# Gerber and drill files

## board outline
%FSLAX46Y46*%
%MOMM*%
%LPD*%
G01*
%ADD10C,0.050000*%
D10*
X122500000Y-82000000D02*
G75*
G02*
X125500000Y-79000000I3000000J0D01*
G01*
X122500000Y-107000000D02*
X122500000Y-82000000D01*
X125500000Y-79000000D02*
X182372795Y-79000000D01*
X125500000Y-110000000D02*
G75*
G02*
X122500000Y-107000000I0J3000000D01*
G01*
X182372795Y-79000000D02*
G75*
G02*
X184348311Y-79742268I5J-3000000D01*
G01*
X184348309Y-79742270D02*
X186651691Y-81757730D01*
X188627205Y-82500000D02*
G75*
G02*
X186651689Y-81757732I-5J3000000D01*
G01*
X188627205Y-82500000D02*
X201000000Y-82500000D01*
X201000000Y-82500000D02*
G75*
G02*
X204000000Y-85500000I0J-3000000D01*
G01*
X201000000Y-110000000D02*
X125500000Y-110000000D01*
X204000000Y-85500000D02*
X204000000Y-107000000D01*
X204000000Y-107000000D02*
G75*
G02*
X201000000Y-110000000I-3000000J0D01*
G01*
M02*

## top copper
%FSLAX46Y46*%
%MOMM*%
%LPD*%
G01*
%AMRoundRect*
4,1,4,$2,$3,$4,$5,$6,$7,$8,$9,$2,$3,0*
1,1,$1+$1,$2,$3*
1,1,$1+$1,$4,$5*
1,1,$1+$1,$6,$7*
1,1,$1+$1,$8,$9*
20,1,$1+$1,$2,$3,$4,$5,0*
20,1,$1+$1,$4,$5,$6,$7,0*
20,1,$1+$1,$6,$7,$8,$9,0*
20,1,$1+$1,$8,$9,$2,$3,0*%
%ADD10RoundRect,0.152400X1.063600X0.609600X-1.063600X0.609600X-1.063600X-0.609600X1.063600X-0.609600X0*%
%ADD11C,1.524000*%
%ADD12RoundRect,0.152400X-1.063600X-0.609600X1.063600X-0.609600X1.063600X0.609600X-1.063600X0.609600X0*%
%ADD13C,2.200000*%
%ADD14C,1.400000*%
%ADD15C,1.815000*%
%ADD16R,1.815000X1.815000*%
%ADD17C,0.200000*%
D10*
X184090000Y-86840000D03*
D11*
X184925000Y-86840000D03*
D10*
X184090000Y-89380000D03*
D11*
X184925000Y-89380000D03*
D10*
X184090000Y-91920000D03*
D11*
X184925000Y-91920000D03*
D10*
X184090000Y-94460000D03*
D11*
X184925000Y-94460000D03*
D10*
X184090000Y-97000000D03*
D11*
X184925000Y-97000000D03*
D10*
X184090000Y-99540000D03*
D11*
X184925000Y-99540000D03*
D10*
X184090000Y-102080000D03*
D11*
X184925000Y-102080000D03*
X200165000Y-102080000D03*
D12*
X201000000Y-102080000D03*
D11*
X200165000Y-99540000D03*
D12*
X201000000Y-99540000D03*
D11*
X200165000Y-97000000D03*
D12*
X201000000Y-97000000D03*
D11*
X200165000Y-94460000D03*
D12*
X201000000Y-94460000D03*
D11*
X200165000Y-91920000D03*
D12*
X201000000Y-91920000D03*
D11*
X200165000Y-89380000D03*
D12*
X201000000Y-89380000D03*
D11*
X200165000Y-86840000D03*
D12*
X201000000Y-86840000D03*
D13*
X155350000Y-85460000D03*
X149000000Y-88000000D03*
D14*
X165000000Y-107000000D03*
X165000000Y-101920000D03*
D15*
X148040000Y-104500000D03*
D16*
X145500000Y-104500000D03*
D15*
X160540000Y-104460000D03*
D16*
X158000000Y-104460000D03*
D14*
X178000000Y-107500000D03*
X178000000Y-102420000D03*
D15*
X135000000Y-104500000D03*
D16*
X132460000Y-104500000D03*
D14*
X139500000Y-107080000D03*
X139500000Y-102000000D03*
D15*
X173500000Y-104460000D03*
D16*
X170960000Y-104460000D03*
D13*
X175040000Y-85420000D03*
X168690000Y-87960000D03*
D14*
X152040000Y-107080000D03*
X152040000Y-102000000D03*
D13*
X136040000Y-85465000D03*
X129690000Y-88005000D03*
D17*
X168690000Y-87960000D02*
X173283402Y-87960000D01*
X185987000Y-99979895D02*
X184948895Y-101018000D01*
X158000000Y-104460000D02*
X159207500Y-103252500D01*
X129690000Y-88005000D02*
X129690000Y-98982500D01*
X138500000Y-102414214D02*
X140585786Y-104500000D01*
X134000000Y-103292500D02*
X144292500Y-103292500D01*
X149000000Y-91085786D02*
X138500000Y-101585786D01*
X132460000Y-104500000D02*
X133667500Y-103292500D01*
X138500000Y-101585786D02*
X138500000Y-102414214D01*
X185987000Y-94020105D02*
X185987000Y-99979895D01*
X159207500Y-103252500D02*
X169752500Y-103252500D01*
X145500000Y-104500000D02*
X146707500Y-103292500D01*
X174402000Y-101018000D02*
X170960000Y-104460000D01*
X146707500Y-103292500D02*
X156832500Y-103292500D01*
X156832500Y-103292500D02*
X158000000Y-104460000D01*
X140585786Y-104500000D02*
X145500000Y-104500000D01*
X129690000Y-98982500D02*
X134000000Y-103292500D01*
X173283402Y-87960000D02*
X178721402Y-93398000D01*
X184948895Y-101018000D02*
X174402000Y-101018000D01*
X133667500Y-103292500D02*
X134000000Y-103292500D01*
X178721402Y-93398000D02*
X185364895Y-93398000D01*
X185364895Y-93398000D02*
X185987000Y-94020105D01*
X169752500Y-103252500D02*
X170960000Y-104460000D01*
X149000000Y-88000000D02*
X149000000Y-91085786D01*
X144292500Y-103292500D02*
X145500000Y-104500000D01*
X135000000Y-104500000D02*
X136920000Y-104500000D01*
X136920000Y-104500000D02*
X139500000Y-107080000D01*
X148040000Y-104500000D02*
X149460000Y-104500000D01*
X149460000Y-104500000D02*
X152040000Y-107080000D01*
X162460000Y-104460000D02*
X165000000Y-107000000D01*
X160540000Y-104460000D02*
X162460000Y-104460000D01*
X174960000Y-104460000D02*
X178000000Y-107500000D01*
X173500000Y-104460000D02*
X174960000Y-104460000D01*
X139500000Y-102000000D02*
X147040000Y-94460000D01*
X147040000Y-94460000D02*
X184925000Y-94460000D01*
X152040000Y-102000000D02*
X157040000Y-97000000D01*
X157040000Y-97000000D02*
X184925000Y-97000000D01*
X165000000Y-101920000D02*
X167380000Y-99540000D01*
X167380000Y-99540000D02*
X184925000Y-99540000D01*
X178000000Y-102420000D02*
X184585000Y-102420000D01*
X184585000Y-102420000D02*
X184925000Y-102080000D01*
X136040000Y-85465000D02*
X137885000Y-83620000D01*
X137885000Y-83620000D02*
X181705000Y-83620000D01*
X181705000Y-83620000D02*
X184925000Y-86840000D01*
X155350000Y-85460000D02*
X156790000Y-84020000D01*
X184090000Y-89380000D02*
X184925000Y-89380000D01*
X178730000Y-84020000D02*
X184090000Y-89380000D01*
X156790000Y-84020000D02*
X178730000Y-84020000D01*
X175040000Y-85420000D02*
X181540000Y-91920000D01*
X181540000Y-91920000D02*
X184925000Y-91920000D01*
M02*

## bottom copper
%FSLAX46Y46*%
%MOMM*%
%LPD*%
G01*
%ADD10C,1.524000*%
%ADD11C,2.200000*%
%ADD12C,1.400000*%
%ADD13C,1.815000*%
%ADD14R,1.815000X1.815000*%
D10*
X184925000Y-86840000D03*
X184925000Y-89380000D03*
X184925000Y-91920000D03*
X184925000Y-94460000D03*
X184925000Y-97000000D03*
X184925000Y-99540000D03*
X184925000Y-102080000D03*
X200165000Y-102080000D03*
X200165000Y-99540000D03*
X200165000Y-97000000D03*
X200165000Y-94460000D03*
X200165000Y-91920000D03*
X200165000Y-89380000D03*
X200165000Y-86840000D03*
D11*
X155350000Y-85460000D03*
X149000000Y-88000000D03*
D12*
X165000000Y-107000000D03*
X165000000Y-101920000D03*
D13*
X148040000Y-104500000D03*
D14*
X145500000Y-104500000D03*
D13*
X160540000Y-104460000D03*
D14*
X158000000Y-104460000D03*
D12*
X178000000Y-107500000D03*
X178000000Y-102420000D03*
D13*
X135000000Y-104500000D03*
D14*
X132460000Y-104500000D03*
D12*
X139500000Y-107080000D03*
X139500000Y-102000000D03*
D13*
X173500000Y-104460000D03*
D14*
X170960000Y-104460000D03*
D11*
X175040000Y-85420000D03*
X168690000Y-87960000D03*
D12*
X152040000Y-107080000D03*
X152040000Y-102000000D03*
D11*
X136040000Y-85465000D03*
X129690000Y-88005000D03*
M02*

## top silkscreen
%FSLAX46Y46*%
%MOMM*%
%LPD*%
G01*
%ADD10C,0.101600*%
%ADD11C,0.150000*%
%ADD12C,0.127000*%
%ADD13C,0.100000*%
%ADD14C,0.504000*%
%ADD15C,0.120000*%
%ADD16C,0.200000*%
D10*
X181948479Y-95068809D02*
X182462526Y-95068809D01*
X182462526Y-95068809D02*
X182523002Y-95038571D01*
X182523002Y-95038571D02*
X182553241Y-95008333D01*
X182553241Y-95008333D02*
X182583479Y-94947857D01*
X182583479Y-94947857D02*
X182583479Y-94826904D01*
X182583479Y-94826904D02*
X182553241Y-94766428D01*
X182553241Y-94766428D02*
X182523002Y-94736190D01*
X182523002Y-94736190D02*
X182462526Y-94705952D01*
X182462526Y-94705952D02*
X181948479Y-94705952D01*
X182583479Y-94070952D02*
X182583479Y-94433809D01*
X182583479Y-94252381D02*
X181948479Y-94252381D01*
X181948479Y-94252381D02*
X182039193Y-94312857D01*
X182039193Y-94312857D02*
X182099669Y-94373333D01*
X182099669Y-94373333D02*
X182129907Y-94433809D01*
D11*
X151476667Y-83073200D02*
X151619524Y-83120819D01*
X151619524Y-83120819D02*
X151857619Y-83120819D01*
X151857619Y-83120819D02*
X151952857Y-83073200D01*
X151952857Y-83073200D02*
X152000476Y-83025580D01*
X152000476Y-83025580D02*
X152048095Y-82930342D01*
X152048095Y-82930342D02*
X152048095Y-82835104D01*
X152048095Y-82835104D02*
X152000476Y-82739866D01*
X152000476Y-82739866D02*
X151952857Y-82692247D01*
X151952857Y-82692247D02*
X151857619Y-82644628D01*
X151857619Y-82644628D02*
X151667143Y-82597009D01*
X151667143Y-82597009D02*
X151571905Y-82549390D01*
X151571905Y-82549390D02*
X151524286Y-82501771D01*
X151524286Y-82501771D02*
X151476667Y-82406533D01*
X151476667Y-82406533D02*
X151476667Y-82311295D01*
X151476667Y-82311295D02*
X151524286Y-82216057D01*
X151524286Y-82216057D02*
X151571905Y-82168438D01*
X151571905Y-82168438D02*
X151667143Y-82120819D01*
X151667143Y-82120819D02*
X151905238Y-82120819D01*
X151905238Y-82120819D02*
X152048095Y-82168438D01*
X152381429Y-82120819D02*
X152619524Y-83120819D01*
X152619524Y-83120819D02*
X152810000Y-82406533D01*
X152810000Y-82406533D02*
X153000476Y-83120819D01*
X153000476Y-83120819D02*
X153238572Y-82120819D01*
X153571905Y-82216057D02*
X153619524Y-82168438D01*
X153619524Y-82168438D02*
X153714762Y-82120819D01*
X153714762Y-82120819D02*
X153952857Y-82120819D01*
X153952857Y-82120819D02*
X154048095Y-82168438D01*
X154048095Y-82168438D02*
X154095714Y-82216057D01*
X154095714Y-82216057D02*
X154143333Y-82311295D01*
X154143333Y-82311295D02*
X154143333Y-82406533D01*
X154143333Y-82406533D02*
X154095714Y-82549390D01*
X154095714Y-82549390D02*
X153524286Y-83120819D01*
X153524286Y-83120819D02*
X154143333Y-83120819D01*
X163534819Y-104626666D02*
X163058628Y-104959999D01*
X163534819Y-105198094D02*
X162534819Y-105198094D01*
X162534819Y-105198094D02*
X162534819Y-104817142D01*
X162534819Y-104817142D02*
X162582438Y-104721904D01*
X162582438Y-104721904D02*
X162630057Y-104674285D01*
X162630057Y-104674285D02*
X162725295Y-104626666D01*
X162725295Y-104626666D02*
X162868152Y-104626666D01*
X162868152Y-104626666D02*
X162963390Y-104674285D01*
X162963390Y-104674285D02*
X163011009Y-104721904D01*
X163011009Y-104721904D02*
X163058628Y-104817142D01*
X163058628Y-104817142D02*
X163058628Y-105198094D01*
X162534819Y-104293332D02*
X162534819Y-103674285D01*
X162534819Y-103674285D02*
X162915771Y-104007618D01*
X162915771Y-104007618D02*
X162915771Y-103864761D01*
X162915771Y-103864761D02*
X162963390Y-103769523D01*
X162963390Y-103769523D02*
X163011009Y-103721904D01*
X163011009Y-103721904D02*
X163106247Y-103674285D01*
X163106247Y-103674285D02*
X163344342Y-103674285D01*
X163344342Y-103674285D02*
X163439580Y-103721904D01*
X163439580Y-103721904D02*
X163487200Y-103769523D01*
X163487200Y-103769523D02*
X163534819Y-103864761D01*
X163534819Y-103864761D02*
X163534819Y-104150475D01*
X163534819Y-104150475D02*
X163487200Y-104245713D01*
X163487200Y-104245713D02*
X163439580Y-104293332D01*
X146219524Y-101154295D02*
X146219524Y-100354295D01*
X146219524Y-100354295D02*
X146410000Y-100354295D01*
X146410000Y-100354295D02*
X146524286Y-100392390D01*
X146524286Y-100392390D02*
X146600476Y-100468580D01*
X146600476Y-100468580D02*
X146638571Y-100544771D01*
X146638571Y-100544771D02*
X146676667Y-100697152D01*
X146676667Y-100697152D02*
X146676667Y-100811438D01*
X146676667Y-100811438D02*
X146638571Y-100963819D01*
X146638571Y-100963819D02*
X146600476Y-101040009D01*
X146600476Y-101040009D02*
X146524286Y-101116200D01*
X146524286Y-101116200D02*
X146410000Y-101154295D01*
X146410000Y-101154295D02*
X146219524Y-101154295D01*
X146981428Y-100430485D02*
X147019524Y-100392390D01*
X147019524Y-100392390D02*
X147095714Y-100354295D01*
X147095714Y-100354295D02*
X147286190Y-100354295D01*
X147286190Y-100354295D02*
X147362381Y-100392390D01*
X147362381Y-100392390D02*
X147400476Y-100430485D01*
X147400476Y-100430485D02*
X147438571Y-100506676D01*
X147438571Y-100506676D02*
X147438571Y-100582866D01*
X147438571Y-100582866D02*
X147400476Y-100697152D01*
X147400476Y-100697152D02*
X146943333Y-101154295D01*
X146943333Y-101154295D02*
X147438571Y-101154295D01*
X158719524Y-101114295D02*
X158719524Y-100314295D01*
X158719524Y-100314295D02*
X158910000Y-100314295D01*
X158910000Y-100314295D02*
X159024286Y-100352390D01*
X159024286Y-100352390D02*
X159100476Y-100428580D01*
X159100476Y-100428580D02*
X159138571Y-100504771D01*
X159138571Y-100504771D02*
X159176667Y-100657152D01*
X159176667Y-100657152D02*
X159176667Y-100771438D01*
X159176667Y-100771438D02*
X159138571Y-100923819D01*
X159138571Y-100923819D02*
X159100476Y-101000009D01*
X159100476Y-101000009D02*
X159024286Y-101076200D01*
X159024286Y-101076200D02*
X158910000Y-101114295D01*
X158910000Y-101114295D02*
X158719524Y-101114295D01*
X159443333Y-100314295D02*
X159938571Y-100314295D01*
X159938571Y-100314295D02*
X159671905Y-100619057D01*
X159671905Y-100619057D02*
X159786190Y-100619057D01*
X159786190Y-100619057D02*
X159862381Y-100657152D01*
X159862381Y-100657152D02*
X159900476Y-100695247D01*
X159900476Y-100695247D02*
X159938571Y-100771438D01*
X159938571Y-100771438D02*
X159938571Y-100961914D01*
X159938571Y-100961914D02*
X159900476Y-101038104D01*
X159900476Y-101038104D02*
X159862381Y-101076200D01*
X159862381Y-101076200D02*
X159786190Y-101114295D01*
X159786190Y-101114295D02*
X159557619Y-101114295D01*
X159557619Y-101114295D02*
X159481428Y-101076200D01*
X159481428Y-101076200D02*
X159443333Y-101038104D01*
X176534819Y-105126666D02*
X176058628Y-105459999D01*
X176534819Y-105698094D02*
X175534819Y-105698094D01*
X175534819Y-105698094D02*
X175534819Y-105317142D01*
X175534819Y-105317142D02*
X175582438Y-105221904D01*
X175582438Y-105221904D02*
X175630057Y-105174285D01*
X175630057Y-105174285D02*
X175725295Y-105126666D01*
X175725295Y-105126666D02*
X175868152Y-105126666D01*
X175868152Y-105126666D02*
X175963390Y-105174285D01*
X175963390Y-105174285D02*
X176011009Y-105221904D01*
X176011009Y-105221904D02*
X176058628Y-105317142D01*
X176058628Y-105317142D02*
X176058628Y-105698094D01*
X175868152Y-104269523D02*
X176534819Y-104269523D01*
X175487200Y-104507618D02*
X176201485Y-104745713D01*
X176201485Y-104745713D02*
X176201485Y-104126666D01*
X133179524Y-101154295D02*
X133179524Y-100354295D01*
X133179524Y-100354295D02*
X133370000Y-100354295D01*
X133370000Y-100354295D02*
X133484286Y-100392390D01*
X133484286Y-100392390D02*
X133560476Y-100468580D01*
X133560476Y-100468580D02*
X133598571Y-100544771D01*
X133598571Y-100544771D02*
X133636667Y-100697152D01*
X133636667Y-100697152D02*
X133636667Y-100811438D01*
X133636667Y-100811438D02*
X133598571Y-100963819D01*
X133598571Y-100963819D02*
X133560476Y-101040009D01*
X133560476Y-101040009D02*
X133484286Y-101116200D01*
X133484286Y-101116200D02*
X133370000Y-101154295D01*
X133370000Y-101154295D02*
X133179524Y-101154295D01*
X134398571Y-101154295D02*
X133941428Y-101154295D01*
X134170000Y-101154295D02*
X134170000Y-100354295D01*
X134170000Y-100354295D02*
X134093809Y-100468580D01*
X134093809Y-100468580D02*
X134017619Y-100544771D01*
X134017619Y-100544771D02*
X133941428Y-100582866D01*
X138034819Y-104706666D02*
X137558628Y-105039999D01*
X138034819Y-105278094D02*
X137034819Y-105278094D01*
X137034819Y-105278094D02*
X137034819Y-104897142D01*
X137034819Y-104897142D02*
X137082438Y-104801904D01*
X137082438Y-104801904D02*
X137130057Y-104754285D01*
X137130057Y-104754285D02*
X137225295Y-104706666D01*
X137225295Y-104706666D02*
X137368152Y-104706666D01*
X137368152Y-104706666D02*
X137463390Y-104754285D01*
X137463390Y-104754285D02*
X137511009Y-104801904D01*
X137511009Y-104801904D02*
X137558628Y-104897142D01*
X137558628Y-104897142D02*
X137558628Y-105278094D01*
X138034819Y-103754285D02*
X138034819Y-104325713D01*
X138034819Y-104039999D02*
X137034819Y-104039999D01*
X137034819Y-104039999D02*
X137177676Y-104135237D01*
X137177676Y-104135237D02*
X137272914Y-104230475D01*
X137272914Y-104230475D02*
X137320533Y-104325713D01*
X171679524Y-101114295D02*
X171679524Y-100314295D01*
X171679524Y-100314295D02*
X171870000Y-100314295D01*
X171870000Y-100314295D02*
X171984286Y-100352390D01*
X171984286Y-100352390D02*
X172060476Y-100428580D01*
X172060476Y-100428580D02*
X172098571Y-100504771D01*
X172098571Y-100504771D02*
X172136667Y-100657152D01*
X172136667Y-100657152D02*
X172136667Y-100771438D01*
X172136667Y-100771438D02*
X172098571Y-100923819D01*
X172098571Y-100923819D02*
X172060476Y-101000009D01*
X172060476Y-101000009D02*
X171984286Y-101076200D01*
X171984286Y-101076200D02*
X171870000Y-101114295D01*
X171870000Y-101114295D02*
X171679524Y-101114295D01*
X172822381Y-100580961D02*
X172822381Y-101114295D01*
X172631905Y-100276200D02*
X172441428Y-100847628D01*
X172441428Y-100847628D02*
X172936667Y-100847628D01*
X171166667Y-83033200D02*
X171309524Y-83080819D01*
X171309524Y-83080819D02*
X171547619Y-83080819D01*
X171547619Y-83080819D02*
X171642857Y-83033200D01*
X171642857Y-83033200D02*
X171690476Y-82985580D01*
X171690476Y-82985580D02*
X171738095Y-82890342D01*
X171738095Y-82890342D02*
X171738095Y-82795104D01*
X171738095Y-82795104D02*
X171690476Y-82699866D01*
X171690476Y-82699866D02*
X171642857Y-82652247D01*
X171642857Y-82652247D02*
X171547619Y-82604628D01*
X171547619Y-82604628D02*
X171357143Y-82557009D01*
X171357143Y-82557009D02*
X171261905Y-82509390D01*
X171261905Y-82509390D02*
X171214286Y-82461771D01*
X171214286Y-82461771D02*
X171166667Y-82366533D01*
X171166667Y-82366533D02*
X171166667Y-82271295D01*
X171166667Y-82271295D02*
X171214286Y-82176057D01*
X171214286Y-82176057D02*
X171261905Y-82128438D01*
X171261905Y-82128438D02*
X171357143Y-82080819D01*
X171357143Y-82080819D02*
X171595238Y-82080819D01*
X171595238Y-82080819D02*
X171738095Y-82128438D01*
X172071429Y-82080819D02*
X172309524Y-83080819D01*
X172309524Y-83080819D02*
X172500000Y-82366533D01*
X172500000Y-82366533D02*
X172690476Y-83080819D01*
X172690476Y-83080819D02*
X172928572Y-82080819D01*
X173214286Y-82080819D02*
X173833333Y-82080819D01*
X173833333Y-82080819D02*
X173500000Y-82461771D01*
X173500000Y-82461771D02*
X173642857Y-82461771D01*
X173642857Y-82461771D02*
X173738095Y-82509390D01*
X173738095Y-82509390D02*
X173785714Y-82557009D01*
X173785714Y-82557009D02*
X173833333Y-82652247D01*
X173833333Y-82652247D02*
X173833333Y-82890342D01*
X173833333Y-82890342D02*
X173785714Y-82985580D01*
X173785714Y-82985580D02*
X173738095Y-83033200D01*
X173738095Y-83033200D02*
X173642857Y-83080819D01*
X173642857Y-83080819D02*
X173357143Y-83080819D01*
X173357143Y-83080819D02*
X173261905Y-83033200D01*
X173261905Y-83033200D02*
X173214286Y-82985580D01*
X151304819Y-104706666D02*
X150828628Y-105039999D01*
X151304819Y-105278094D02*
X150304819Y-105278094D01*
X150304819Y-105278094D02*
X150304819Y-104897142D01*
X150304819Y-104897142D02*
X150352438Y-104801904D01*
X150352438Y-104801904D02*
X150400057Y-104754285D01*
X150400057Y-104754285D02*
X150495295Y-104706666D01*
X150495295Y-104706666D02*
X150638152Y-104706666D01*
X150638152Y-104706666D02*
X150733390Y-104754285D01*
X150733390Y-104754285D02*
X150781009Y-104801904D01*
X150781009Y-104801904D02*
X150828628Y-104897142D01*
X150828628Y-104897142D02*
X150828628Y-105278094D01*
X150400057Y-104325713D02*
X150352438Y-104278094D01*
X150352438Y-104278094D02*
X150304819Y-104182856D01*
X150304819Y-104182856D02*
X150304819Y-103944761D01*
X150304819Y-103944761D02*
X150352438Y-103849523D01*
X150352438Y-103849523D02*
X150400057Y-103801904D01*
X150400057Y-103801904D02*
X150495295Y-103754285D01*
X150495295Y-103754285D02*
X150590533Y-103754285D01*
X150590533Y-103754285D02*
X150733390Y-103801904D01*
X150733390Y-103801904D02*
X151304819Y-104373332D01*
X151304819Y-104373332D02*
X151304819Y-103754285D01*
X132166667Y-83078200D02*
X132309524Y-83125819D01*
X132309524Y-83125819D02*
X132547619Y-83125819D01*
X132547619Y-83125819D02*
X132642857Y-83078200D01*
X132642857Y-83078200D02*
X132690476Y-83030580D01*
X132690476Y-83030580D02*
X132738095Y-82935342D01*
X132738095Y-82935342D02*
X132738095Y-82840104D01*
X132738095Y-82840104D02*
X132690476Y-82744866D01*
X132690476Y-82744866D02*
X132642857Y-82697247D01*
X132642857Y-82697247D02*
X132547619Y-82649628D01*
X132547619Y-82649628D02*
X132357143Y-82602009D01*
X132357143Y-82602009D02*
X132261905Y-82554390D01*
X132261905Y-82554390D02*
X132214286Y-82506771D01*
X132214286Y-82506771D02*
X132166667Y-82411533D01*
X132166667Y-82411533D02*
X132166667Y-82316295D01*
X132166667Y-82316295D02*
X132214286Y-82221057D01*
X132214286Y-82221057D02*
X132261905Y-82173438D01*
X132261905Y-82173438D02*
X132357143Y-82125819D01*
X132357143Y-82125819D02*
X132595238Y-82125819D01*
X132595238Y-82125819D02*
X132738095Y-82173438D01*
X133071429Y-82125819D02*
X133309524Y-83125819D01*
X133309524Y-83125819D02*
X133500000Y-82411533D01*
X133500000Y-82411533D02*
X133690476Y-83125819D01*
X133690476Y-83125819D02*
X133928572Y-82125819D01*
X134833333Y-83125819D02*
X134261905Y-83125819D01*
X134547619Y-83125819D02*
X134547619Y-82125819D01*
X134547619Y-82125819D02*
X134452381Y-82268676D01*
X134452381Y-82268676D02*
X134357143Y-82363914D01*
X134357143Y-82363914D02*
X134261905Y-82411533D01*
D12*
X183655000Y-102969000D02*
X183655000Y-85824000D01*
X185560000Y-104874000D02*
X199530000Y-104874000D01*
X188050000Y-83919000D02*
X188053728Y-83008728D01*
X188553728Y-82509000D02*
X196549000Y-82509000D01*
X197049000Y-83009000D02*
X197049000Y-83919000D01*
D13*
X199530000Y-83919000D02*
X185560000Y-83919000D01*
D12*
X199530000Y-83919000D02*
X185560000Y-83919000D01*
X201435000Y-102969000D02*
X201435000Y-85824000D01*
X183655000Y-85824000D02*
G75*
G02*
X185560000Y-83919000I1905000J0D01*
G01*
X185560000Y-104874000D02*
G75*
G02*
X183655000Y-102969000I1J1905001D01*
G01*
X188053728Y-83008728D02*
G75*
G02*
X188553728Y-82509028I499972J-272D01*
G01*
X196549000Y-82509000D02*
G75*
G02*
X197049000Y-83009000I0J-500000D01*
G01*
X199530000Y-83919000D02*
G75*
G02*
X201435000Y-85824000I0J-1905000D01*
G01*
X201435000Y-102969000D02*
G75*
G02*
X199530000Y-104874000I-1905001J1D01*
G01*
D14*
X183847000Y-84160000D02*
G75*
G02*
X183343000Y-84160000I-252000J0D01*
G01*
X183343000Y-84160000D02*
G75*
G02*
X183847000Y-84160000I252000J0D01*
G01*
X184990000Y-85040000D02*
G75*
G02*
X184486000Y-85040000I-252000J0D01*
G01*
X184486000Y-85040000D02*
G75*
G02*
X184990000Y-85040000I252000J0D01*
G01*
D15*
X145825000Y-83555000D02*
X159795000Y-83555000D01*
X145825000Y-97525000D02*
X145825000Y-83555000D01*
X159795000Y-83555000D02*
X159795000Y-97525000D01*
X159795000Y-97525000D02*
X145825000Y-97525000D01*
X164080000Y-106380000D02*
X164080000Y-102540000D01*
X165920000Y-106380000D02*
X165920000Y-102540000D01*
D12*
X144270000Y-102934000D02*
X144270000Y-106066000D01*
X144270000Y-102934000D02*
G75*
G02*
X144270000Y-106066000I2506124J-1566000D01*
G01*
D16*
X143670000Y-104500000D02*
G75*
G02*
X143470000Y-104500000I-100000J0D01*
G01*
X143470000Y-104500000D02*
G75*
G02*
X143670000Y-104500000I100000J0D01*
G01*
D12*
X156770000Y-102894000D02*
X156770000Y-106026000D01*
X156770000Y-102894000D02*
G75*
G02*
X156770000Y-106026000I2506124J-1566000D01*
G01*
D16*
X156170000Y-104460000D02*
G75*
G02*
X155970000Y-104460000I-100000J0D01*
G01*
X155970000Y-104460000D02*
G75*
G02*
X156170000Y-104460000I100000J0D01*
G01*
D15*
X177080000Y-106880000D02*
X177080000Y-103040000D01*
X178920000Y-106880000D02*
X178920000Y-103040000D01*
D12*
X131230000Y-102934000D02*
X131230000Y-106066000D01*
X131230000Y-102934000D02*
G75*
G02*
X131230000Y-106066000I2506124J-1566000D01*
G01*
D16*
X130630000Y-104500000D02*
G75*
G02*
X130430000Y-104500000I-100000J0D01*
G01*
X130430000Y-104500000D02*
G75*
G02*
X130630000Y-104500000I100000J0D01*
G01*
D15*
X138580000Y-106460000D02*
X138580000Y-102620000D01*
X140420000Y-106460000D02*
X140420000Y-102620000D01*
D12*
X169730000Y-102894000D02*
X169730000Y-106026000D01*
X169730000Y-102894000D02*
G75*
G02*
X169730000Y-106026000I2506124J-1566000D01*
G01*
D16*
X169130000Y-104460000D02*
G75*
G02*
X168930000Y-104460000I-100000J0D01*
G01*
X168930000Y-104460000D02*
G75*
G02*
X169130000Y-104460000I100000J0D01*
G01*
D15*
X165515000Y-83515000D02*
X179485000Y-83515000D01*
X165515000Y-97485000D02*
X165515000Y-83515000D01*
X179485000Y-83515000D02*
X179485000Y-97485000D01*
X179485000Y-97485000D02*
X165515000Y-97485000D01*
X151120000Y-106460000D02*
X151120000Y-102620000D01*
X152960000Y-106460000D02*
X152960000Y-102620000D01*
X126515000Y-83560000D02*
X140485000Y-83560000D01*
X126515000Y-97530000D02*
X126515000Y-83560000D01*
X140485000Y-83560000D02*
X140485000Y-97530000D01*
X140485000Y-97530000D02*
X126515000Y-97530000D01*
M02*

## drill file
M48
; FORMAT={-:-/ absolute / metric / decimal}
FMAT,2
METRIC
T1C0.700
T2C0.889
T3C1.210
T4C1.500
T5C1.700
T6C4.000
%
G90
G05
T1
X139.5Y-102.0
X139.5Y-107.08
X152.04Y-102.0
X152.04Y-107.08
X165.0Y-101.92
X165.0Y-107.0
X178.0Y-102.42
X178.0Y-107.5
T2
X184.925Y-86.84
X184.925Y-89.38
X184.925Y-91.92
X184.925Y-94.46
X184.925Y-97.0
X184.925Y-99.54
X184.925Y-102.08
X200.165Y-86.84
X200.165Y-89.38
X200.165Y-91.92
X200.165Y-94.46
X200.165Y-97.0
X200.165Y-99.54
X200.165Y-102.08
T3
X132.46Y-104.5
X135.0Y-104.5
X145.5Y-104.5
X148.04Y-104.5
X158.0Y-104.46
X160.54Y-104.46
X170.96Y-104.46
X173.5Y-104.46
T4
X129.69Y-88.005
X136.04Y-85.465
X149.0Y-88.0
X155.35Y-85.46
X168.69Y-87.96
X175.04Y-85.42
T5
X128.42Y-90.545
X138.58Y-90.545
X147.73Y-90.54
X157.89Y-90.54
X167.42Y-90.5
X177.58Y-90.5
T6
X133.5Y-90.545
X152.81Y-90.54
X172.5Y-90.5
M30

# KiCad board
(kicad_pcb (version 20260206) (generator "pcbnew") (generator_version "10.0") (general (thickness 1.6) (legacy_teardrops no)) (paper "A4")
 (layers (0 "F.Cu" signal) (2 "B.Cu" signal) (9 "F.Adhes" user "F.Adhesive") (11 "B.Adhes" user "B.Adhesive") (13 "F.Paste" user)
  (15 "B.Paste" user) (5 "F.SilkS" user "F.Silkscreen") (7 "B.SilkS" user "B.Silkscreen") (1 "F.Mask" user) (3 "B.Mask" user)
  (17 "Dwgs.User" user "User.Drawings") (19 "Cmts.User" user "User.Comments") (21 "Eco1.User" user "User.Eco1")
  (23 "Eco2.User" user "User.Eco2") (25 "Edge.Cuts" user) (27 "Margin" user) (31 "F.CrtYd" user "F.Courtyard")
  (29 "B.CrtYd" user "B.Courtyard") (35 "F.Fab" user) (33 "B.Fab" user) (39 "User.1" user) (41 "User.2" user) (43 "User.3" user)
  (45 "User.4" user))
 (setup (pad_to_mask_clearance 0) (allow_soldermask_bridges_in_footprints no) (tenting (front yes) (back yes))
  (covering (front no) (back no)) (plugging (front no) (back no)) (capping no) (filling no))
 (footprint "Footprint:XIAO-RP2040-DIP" (layer "F.Cu") (at 192.545 94.46 90)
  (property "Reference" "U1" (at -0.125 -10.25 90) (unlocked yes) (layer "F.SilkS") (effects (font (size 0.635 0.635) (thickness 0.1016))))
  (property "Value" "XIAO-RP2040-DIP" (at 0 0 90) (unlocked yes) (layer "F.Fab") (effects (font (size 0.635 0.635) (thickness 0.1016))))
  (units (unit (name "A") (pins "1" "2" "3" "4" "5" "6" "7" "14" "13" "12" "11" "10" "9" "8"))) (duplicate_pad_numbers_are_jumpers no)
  (fp_line (start -8.509 -8.89) (end 8.636 -8.89) (stroke (width 0.127) (type solid)) (layer "F.SilkS"))
  (fp_line (start -10.414 -6.985) (end -10.414 6.985) (stroke (width 0.127) (type solid)) (layer "F.SilkS"))
  (fp_line (start 10.541 -4.495) (end 11.451272 -4.491272) (stroke (width 0.127) (type solid)) (layer "F.SilkS"))
  (fp_line (start 11.951 -3.991272) (end 11.951 4.004) (stroke (width 0.127) (type solid)) (layer "F.SilkS"))
  (fp_line (start 11.451 4.504) (end 10.541 4.504) (stroke (width 0.127) (type solid)) (layer "F.SilkS"))
  (fp_line (start 10.541 6.985) (end 10.541 -6.985) (stroke (width 0.1) (type solid)) (layer "F.SilkS"))
  (fp_line (start 10.541 6.985) (end 10.541 -6.985) (stroke (width 0.127) (type solid)) (layer "F.SilkS"))
  (fp_line (start -8.509 8.89) (end 8.636 8.89) (stroke (width 0.127) (type solid)) (layer "F.SilkS"))
  (fp_arc (start 8.636 -8.89) (mid 9.983038 -8.332038) (end 10.541 -6.985) (stroke (width 0.127) (type solid)) (layer "F.SilkS"))
  (fp_arc (start -10.414 -6.985) (mid -9.856038 -8.332038) (end -8.509 -8.89) (stroke (width 0.127) (type solid)) (layer "F.SilkS"))
  (fp_arc (start 11.451272 -4.491272) (mid 11.804644 -4.344724) (end 11.951 -3.991272) (stroke (width 0.127) (type default))
   (layer "F.SilkS"))
  (fp_arc (start 11.951 4.004) (mid 11.804553 4.357553) (end 11.451 4.504) (stroke (width 0.127) (type default)) (layer "F.SilkS"))
  (fp_arc (start 10.541 6.985) (mid 9.983038 8.332038) (end 8.636 8.89) (stroke (width 0.127) (type solid)) (layer "F.SilkS"))
  (fp_arc (start -8.509 8.89) (mid -9.856038 8.332038) (end -10.414 6.985) (stroke (width 0.127) (type solid)) (layer "F.SilkS"))
  (fp_circle (center 10.3 -8.95) (end 10.554 -8.95) (stroke (width 0.5) (type solid)) (fill yes) (layer "F.SilkS"))
  (fp_circle (center 9.42 -7.807) (end 9.674 -7.807) (stroke (width 0.5) (type solid)) (fill yes) (layer "F.SilkS"))
  (pad "1" smd roundrect (at 7.62 -8.455 180) (size 2.432 1.524) (layers "F.Cu" "F.Mask") (roundrect_rratio 0.1) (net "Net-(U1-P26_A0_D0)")
   (thermal_bridge_angle 45))
  (pad "1" thru_hole circle (at 7.62 -7.62 180) (size 1.524 1.524) (drill 0.889) (layers "*.Cu" "*.Mask") (remove_unused_layers no)
   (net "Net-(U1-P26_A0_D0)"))
  (pad "2" smd roundrect (at 5.08 -8.455 180) (size 2.432 1.524) (layers "F.Cu" "F.Mask") (roundrect_rratio 0.1) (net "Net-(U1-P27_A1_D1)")
   (thermal_bridge_angle 45))
  (pad "2" thru_hole circle (at 5.08 -7.62 180) (size 1.524 1.524) (drill 0.889) (layers "*.Cu" "*.Mask") (remove_unused_layers no)
   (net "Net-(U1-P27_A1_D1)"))
  (pad "3" smd roundrect (at 2.54 -8.455 180) (size 2.432 1.524) (layers "F.Cu" "F.Mask") (roundrect_rratio 0.1) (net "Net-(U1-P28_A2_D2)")
   (thermal_bridge_angle 45))
  (pad "3" thru_hole circle (at 2.54 -7.62 180) (size 1.524 1.524) (drill 0.889) (layers "*.Cu" "*.Mask") (remove_unused_layers no)
   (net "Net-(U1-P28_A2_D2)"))
  (pad "4" smd roundrect (at 0 -8.455 180) (size 2.432 1.524) (layers "F.Cu" "F.Mask") (roundrect_rratio 0.1) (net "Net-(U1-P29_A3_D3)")
   (thermal_bridge_angle 45))
  (pad "4" thru_hole circle (at 0 -7.62 180) (size 1.524 1.524) (drill 0.889) (layers "*.Cu" "*.Mask") (remove_unused_layers no)
   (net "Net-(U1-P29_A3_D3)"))
  (pad "5" smd roundrect (at -2.54 -8.455 180) (size 2.432 1.524) (layers "F.Cu" "F.Mask") (roundrect_rratio 0.1) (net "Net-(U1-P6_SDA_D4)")
   (thermal_bridge_angle 45))
  (pad "5" thru_hole circle (at -2.54 -7.62 180) (size 1.524 1.524) (drill 0.889) (layers "*.Cu" "*.Mask") (remove_unused_layers no)
   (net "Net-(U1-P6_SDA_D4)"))
  (pad "6" smd roundrect (at -5.08 -8.455 180) (size 2.432 1.524) (layers "F.Cu" "F.Mask") (roundrect_rratio 0.1) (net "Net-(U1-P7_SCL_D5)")
   (thermal_bridge_angle 45))
  (pad "6" thru_hole circle (at -5.08 -7.62 180) (size 1.524 1.524) (drill 0.889) (layers "*.Cu" "*.Mask") (remove_unused_layers no)
   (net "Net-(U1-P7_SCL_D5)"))
  (pad "7" smd roundrect (at -7.62 -8.455 180) (size 2.432 1.524) (layers "F.Cu" "F.Mask") (roundrect_rratio 0.1) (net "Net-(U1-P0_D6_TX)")
   (thermal_bridge_angle 45))
  (pad "7" thru_hole circle (at -7.62 -7.62 180) (size 1.524 1.524) (drill 0.889) (layers "*.Cu" "*.Mask") (remove_unused_layers no)
   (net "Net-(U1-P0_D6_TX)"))
  (pad "8" thru_hole circle (at -7.62 7.62) (size 1.524 1.524) (drill 0.889) (layers "*.Cu" "*.Mask") (remove_unused_layers no)
   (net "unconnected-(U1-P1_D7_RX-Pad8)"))
  (pad "8" smd roundrect (at -7.62 8.455) (size 2.432 1.524) (layers "F.Cu" "F.Mask") (roundrect_rratio 0.1)
   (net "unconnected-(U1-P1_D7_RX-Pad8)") (thermal_bridge_angle 45))
  (pad "9" thru_hole circle (at -5.08 7.62) (size 1.524 1.524) (drill 0.889) (layers "*.Cu" "*.Mask") (remove_unused_layers no)
   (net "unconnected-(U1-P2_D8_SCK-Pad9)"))
  (pad "9" smd roundrect (at -5.08 8.455) (size 2.432 1.524) (layers "F.Cu" "F.Mask") (roundrect_rratio 0.1)
   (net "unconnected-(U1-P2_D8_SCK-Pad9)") (thermal_bridge_angle 45))
  (pad "10" thru_hole circle (at -2.54 7.62) (size 1.524 1.524) (drill 0.889) (layers "*.Cu" "*.Mask") (remove_unused_layers no)
   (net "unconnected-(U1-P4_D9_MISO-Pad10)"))
  (pad "10" smd roundrect (at -2.54 8.455) (size 2.432 1.524) (layers "F.Cu" "F.Mask") (roundrect_rratio 0.1)
   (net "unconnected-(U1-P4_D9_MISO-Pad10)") (thermal_bridge_angle 45))
  (pad "11" thru_hole circle (at 0 7.62) (size 1.524 1.524) (drill 0.889) (layers "*.Cu" "*.Mask") (remove_unused_layers no)
   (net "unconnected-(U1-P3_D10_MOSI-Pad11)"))
  (pad "11" smd roundrect (at 0 8.455) (size 2.432 1.524) (layers "F.Cu" "F.Mask") (roundrect_rratio 0.1)
   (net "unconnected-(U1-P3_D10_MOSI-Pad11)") (thermal_bridge_angle 45))
  (pad "12" thru_hole circle (at 2.54 7.62) (size 1.524 1.524) (drill 0.889) (layers "*.Cu" "*.Mask") (remove_unused_layers no)
   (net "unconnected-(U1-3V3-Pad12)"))
  (pad "12" smd roundrect (at 2.54 8.455) (size 2.432 1.524) (layers "F.Cu" "F.Mask") (roundrect_rratio 0.1)
   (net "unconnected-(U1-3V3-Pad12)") (thermal_bridge_angle 45))
  (pad "13" thru_hole circle (at 5.08 7.62) (size 1.524 1.524) (drill 0.889) (layers "*.Cu" "*.Mask") (remove_unused_layers no)
   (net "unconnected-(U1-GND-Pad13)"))
  (pad "13" smd roundrect (at 5.08 8.455) (size 2.432 1.524) (layers "F.Cu" "F.Mask") (roundrect_rratio 0.1)
   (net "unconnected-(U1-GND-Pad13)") (thermal_bridge_angle 45))
  (pad "14" thru_hole circle (at 7.62 7.62) (size 1.524 1.524) (drill 0.889) (layers "*.Cu" "*.Mask") (remove_unused_layers no)
   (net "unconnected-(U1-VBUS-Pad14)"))
  (pad "14" smd roundrect (at 7.62 8.455) (size 2.432 1.524) (layers "F.Cu" "F.Mask") (roundrect_rratio 0.1)
   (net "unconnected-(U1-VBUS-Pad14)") (thermal_bridge_angle 45)))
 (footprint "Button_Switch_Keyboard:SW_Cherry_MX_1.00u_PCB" (layer "F.Cu") (at 155.35 85.46)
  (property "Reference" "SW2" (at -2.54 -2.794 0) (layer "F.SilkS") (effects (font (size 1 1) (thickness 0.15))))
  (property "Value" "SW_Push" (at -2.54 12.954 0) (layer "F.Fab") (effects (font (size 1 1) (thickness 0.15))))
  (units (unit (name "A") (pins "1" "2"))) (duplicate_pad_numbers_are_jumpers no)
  (fp_line (start -9.525 -1.905) (end 4.445 -1.905) (stroke (width 0.12) (type solid)) (layer "F.SilkS"))
  (fp_line (start -9.525 12.065) (end -9.525 -1.905) (stroke (width 0.12) (type solid)) (layer "F.SilkS"))
  (fp_line (start 4.445 -1.905) (end 4.445 12.065) (stroke (width 0.12) (type solid)) (layer "F.SilkS"))
  (fp_line (start 4.445 12.065) (end -9.525 12.065) (stroke (width 0.12) (type solid)) (layer "F.SilkS"))
  (pad "" np_thru_hole circle (at -7.62 5.08) (size 1.7 1.7) (drill 1.7) (layers "*.Cu" "*.Mask"))
  (pad "" np_thru_hole circle (at -2.54 5.08) (size 4 4) (drill 4) (layers "*.Cu" "*.Mask"))
  (pad "" np_thru_hole circle (at 2.54 5.08) (size 1.7 1.7) (drill 1.7) (layers "*.Cu" "*.Mask"))
  (pad "1" thru_hole circle (at 0 0) (size 2.2 2.2) (drill 1.5) (layers "*.Cu" "*.Mask") (remove_unused_layers no)
   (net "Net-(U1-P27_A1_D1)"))
  (pad "2" thru_hole circle (at -6.35 2.54) (size 2.2 2.2) (drill 1.5) (layers "*.Cu" "*.Mask") (remove_unused_layers no) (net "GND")))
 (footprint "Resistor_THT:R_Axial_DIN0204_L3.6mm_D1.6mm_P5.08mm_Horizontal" (layer "F.Cu") (at 165 107 90)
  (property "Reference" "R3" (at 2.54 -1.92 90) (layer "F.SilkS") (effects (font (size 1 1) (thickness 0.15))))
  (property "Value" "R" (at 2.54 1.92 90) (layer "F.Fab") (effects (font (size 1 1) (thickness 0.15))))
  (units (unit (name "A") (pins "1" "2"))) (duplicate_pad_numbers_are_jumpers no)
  (fp_line (start 0.62 -0.92) (end 4.46 -0.92) (stroke (width 0.12) (type solid)) (layer "F.SilkS"))
  (fp_line (start 0.62 0.92) (end 4.46 0.92) (stroke (width 0.12) (type solid)) (layer "F.SilkS"))
  (pad "1" thru_hole circle (at 0 0 90) (size 1.4 1.4) (drill 0.7) (layers "*.Cu" "*.Mask") (remove_unused_layers no) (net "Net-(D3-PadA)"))
  (pad "2" thru_hole circle (at 5.08 0 90) (size 1.4 1.4) (drill 0.7) (layers "*.Cu" "*.Mask") (remove_unused_layers no)
   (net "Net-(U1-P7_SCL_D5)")))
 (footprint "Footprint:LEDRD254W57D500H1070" (layer "F.Cu") (at 146.77 104.5)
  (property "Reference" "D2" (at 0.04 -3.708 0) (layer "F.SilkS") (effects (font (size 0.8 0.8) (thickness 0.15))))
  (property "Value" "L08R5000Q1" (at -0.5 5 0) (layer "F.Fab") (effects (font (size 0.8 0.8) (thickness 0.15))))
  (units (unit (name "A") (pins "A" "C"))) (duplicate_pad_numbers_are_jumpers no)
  (fp_line (start -2.5 -1.566) (end -2.5 1.566) (stroke (width 0.127) (type solid)) (layer "F.SilkS"))
  (fp_arc (start -2.5 -1.566) (mid 2.961291 0) (end -2.5 1.566) (stroke (width 0.127) (type solid)) (layer "F.SilkS"))
  (fp_circle (center -3.2 0) (end -3.1 0) (stroke (width 0.2) (type solid)) (fill no) (layer "F.SilkS"))
  (pad "A" thru_hole circle (at 1.27 0) (size 1.815 1.815) (drill 1.21) (layers "*.Cu" "*.Mask") (remove_unused_layers no)
   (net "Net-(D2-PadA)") (solder_mask_margin 0.102))
  (pad "C" thru_hole rect (at -1.27 0) (size 1.815 1.815) (drill 1.21) (layers "*.Cu" "*.Mask") (remove_unused_layers no) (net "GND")
   (solder_mask_margin 0.102)))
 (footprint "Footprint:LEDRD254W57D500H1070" (layer "F.Cu") (at 159.27 104.46)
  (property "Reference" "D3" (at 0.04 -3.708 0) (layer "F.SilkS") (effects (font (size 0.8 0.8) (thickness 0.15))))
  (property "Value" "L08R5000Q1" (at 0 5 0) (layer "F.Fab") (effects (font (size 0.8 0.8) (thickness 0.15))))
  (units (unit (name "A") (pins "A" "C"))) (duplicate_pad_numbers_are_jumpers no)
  (fp_line (start -2.5 -1.566) (end -2.5 1.566) (stroke (width 0.127) (type solid)) (layer "F.SilkS"))
  (fp_arc (start -2.5 -1.566) (mid 2.961291 0) (end -2.5 1.566) (stroke (width 0.127) (type solid)) (layer "F.SilkS"))
  (fp_circle (center -3.2 0) (end -3.1 0) (stroke (width 0.2) (type solid)) (fill no) (layer "F.SilkS"))
  (pad "A" thru_hole circle (at 1.27 0) (size 1.815 1.815) (drill 1.21) (layers "*.Cu" "*.Mask") (remove_unused_layers no)
   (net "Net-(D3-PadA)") (solder_mask_margin 0.102))
  (pad "C" thru_hole rect (at -1.27 0) (size 1.815 1.815) (drill 1.21) (layers "*.Cu" "*.Mask") (remove_unused_layers no) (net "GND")
   (solder_mask_margin 0.102)))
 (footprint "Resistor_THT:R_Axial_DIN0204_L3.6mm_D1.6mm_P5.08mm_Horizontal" (layer "F.Cu") (at 178 107.5 90)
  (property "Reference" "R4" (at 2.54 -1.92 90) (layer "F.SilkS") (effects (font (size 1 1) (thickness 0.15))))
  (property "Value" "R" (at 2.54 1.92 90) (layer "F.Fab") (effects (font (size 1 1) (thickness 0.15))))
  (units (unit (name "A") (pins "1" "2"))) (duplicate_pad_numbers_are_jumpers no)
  (fp_line (start 0.62 -0.92) (end 4.46 -0.92) (stroke (width 0.12) (type solid)) (layer "F.SilkS"))
  (fp_line (start 0.62 0.92) (end 4.46 0.92) (stroke (width 0.12) (type solid)) (layer "F.SilkS"))
  (pad "1" thru_hole circle (at 0 0 90) (size 1.4 1.4) (drill 0.7) (layers "*.Cu" "*.Mask") (remove_unused_layers no) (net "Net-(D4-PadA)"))
  (pad "2" thru_hole circle (at 5.08 0 90) (size 1.4 1.4) (drill 0.7) (layers "*.Cu" "*.Mask") (remove_unused_layers no)
   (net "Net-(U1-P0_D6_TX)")))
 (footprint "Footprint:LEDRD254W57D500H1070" (layer "F.Cu") (at 133.73 104.5)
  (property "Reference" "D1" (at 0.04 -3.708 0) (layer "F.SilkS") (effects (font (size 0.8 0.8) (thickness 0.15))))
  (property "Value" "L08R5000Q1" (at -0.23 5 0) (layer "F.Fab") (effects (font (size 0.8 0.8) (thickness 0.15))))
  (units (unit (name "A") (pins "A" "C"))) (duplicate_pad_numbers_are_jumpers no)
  (fp_line (start -2.5 -1.566) (end -2.5 1.566) (stroke (width 0.127) (type solid)) (layer "F.SilkS"))
  (fp_arc (start -2.5 -1.566) (mid 2.961291 0) (end -2.5 1.566) (stroke (width 0.127) (type solid)) (layer "F.SilkS"))
  (fp_circle (center -3.2 0) (end -3.1 0) (stroke (width 0.2) (type solid)) (fill no) (layer "F.SilkS"))
  (pad "A" thru_hole circle (at 1.27 0) (size 1.815 1.815) (drill 1.21) (layers "*.Cu" "*.Mask") (remove_unused_layers no)
   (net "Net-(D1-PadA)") (solder_mask_margin 0.102))
  (pad "C" thru_hole rect (at -1.27 0) (size 1.815 1.815) (drill 1.21) (layers "*.Cu" "*.Mask") (remove_unused_layers no) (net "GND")
   (solder_mask_margin 0.102)))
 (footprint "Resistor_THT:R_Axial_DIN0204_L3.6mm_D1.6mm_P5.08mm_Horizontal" (layer "F.Cu") (at 139.5 107.08 90)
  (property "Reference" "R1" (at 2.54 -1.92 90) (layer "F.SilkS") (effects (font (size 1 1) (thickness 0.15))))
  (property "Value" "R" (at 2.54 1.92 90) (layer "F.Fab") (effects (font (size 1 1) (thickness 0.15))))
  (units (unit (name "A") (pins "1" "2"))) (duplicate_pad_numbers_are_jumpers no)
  (fp_line (start 0.62 -0.92) (end 4.46 -0.92) (stroke (width 0.12) (type solid)) (layer "F.SilkS"))
  (fp_line (start 0.62 0.92) (end 4.46 0.92) (stroke (width 0.12) (type solid)) (layer "F.SilkS"))
  (pad "1" thru_hole circle (at 0 0 90) (size 1.4 1.4) (drill 0.7) (layers "*.Cu" "*.Mask") (remove_unused_layers no) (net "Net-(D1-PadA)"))
  (pad "2" thru_hole circle (at 5.08 0 90) (size 1.4 1.4) (drill 0.7) (layers "*.Cu" "*.Mask") (remove_unused_layers no)
   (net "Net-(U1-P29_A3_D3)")))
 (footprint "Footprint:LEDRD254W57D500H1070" (layer "F.Cu") (at 172.23 104.46)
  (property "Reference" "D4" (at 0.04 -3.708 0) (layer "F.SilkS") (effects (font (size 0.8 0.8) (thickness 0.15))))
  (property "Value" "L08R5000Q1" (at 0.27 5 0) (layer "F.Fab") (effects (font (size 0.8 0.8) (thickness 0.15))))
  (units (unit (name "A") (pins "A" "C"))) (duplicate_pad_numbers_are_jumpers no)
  (fp_line (start -2.5 -1.566) (end -2.5 1.566) (stroke (width 0.127) (type solid)) (layer "F.SilkS"))
  (fp_arc (start -2.5 -1.566) (mid 2.961291 0) (end -2.5 1.566) (stroke (width 0.127) (type solid)) (layer "F.SilkS"))
  (fp_circle (center -3.2 0) (end -3.1 0) (stroke (width 0.2) (type solid)) (fill no) (layer "F.SilkS"))
  (pad "A" thru_hole circle (at 1.27 0) (size 1.815 1.815) (drill 1.21) (layers "*.Cu" "*.Mask") (remove_unused_layers no)
   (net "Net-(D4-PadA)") (solder_mask_margin 0.102))
  (pad "C" thru_hole rect (at -1.27 0) (size 1.815 1.815) (drill 1.21) (layers "*.Cu" "*.Mask") (remove_unused_layers no) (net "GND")
   (solder_mask_margin 0.102)))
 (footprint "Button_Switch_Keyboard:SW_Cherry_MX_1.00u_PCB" (layer "F.Cu") (at 175.04 85.42)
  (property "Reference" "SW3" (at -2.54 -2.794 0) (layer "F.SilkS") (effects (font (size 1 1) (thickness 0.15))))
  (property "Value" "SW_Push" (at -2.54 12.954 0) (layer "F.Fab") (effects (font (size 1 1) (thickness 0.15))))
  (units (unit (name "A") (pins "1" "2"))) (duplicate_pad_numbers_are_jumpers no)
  (fp_line (start -9.525 -1.905) (end 4.445 -1.905) (stroke (width 0.12) (type solid)) (layer "F.SilkS"))
  (fp_line (start -9.525 12.065) (end -9.525 -1.905) (stroke (width 0.12) (type solid)) (layer "F.SilkS"))
  (fp_line (start 4.445 -1.905) (end 4.445 12.065) (stroke (width 0.12) (type solid)) (layer "F.SilkS"))
  (fp_line (start 4.445 12.065) (end -9.525 12.065) (stroke (width 0.12) (type solid)) (layer "F.SilkS"))
  (pad "" np_thru_hole circle (at -7.62 5.08) (size 1.7 1.7) (drill 1.7) (layers "*.Cu" "*.Mask"))
  (pad "" np_thru_hole circle (at -2.54 5.08) (size 4 4) (drill 4) (layers "*.Cu" "*.Mask"))
  (pad "" np_thru_hole circle (at 2.54 5.08) (size 1.7 1.7) (drill 1.7) (layers "*.Cu" "*.Mask"))
  (pad "1" thru_hole circle (at 0 0) (size 2.2 2.2) (drill 1.5) (layers "*.Cu" "*.Mask") (remove_unused_layers no)
   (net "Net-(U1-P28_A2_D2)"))
  (pad "2" thru_hole circle (at -6.35 2.54) (size 2.2 2.2) (drill 1.5) (layers "*.Cu" "*.Mask") (remove_unused_layers no) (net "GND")))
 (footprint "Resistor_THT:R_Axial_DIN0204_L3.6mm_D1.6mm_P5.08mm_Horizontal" (layer "F.Cu") (at 152.04 107.08 90)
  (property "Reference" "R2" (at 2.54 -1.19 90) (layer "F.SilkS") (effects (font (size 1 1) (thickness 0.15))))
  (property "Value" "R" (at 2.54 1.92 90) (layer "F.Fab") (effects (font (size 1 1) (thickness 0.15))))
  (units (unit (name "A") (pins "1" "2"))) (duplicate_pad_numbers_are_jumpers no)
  (fp_line (start 0.62 -0.92) (end 4.46 -0.92) (stroke (width 0.12) (type solid)) (layer "F.SilkS"))
  (fp_line (start 0.62 0.92) (end 4.46 0.92) (stroke (width 0.12) (type solid)) (layer "F.SilkS"))
  (pad "1" thru_hole circle (at 0 0 90) (size 1.4 1.4) (drill 0.7) (layers "*.Cu" "*.Mask") (remove_unused_layers no) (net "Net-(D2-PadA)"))
  (pad "2" thru_hole circle (at 5.08 0 90) (size 1.4 1.4) (drill 0.7) (layers "*.Cu" "*.Mask") (remove_unused_layers no)
   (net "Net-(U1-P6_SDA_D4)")))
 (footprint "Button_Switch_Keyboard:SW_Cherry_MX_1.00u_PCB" (layer "F.Cu") (at 136.04 85.465)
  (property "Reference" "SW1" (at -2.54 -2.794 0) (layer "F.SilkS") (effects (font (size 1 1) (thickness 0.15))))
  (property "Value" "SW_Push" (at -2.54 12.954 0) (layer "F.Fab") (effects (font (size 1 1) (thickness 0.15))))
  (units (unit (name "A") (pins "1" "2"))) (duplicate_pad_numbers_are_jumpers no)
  (fp_line (start -9.525 -1.905) (end 4.445 -1.905) (stroke (width 0.12) (type solid)) (layer "F.SilkS"))
  (fp_line (start -9.525 12.065) (end -9.525 -1.905) (stroke (width 0.12) (type solid)) (layer "F.SilkS"))
  (fp_line (start 4.445 -1.905) (end 4.445 12.065) (stroke (width 0.12) (type solid)) (layer "F.SilkS"))
  (fp_line (start 4.445 12.065) (end -9.525 12.065) (stroke (width 0.12) (type solid)) (layer "F.SilkS"))
  (pad "" np_thru_hole circle (at -7.62 5.08) (size 1.7 1.7) (drill 1.7) (layers "*.Cu" "*.Mask"))
  (pad "" np_thru_hole circle (at -2.54 5.08) (size 4 4) (drill 4) (layers "*.Cu" "*.Mask"))
  (pad "" np_thru_hole circle (at 2.54 5.08) (size 1.7 1.7) (drill 1.7) (layers "*.Cu" "*.Mask"))
  (pad "1" thru_hole circle (at 0 0) (size 2.2 2.2) (drill 1.5) (layers "*.Cu" "*.Mask") (remove_unused_layers no)
   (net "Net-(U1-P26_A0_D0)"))
  (pad "2" thru_hole circle (at -6.35 2.54) (size 2.2 2.2) (drill 1.5) (layers "*.Cu" "*.Mask") (remove_unused_layers no) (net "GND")))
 (gr_arc (start 122.5 82) (mid 123.37868 79.87868) (end 125.5 79) (stroke (width 0.05) (type default)) (layer "Edge.Cuts"))
 (gr_line (start 122.5 107) (end 122.5 82) (stroke (width 0.05) (type default)) (layer "Edge.Cuts"))
 (gr_line (start 125.5 79) (end 182.372795 79) (stroke (width 0.05) (type default)) (layer "Edge.Cuts"))
 (gr_arc (start 125.5 110) (mid 123.37868 109.12132) (end 122.5 107) (stroke (width 0.05) (type default)) (layer "Edge.Cuts"))
 (gr_arc (start 182.372795 79) (mid 183.427975 79.191692) (end 184.348309 79.74227) (stroke (width 0.05) (type default)) (layer "Edge.Cuts"))
 (gr_line (start 184.348309 79.74227) (end 186.651691 81.75773) (stroke (width 0.05) (type default)) (layer "Edge.Cuts"))
 (gr_arc (start 188.627205 82.5) (mid 187.572025 82.308308) (end 186.651691 81.75773) (stroke (width 0.05) (type default))
  (layer "Edge.Cuts"))
 (gr_line (start 188.627205 82.5) (end 201 82.5) (stroke (width 0.05) (type default)) (layer "Edge.Cuts"))
 (gr_arc (start 201 82.5) (mid 203.12132 83.37868) (end 204 85.5) (stroke (width 0.05) (type default)) (layer "Edge.Cuts"))
 (gr_line (start 201 110) (end 125.5 110) (stroke (width 0.05) (type default)) (layer "Edge.Cuts"))
 (gr_line (start 204 85.5) (end 204 107) (stroke (width 0.05) (type default)) (layer "Edge.Cuts"))
 (gr_arc (start 204 107) (mid 203.12132 109.12132) (end 201 110) (stroke (width 0.05) (type default)) (layer "Edge.Cuts"))
 (segment (start 168.69 87.96) (end 173.283402 87.96) (width 0.2) (layer "F.Cu") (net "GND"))
 (segment (start 185.987 99.979895) (end 184.948895 101.018) (width 0.2) (layer "F.Cu") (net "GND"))
 (segment (start 158 104.46) (end 159.2075 103.2525) (width 0.2) (layer "F.Cu") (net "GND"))
 (segment (start 129.69 88.005) (end 129.69 98.9825) (width 0.2) (layer "F.Cu") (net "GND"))
 (segment (start 138.5 102.414214) (end 140.585786 104.5) (width 0.2) (layer "F.Cu") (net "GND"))
 (segment (start 134 103.2925) (end 144.2925 103.2925) (width 0.2) (layer "F.Cu") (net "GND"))
 (segment (start 149 91.085786) (end 138.5 101.585786) (width 0.2) (layer "F.Cu") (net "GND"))
 (segment (start 132.46 104.5) (end 133.6675 103.2925) (width 0.2) (layer "F.Cu") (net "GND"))
 (segment (start 138.5 101.585786) (end 138.5 102.414214) (width 0.2) (layer "F.Cu") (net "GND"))
 (segment (start 185.987 94.020105) (end 185.987 99.979895) (width 0.2) (layer "F.Cu") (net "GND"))
 (segment (start 159.2075 103.2525) (end 169.7525 103.2525) (width 0.2) (layer "F.Cu") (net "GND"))
 (segment (start 145.5 104.5) (end 146.7075 103.2925) (width 0.2) (layer "F.Cu") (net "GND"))
 (segment (start 174.402 101.018) (end 170.96 104.46) (width 0.2) (layer "F.Cu") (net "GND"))
 (segment (start 146.7075 103.2925) (end 156.8325 103.2925) (width 0.2) (layer "F.Cu") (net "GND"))
 (segment (start 156.8325 103.2925) (end 158 104.46) (width 0.2) (layer "F.Cu") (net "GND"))
 (segment (start 140.585786 104.5) (end 145.5 104.5) (width 0.2) (layer "F.Cu") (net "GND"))
 (segment (start 129.69 98.9825) (end 134 103.2925) (width 0.2) (layer "F.Cu") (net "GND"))
 (segment (start 173.283402 87.96) (end 178.721402 93.398) (width 0.2) (layer "F.Cu") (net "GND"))
 (segment (start 184.948895 101.018) (end 174.402 101.018) (width 0.2) (layer "F.Cu") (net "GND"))
 (segment (start 133.6675 103.2925) (end 134 103.2925) (width 0.2) (layer "F.Cu") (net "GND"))
 (segment (start 178.721402 93.398) (end 185.364895 93.398) (width 0.2) (layer "F.Cu") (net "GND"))
 (segment (start 185.364895 93.398) (end 185.987 94.020105) (width 0.2) (layer "F.Cu") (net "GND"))
 (segment (start 169.7525 103.2525) (end 170.96 104.46) (width 0.2) (layer "F.Cu") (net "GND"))
 (segment (start 149 88) (end 149 91.085786) (width 0.2) (layer "F.Cu") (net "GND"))
 (segment (start 144.2925 103.2925) (end 145.5 104.5) (width 0.2) (layer "F.Cu") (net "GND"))
 (segment (start 135 104.5) (end 136.92 104.5) (width 0.2) (layer "F.Cu") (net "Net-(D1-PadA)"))
 (segment (start 136.92 104.5) (end 139.5 107.08) (width 0.2) (layer "F.Cu") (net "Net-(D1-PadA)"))
 (segment (start 148.04 104.5) (end 149.46 104.5) (width 0.2) (layer "F.Cu") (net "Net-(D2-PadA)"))
 (segment (start 149.46 104.5) (end 152.04 107.08) (width 0.2) (layer "F.Cu") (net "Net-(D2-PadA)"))
 (segment (start 162.46 104.46) (end 165 107) (width 0.2) (layer "F.Cu") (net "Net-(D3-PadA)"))
 (segment (start 160.54 104.46) (end 162.46 104.46) (width 0.2) (layer "F.Cu") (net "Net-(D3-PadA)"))
 (segment (start 174.96 104.46) (end 178 107.5) (width 0.2) (layer "F.Cu") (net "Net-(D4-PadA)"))
 (segment (start 173.5 104.46) (end 174.96 104.46) (width 0.2) (layer "F.Cu") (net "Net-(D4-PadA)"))
 (segment (start 139.5 102) (end 147.04 94.46) (width 0.2) (layer "F.Cu") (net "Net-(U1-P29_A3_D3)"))
 (segment (start 147.04 94.46) (end 184.925 94.46) (width 0.2) (layer "F.Cu") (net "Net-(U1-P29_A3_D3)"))
 (segment (start 152.04 102) (end 157.04 97) (width 0.2) (layer "F.Cu") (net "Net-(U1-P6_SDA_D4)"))
 (segment (start 157.04 97) (end 184.925 97) (width 0.2) (layer "F.Cu") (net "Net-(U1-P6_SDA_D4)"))
 (segment (start 165 101.92) (end 167.38 99.54) (width 0.2) (layer "F.Cu") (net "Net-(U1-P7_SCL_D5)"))
 (segment (start 167.38 99.54) (end 184.925 99.54) (width 0.2) (layer "F.Cu") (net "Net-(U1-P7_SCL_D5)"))
 (segment (start 178 102.42) (end 184.585 102.42) (width 0.2) (layer "F.Cu") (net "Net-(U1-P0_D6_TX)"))
 (segment (start 184.585 102.42) (end 184.925 102.08) (width 0.2) (layer "F.Cu") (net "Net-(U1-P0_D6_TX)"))
 (segment (start 136.04 85.465) (end 137.885 83.62) (width 0.2) (layer "F.Cu") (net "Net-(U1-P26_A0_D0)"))
 (segment (start 137.885 83.62) (end 181.705 83.62) (width 0.2) (layer "F.Cu") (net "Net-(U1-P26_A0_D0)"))
 (segment (start 181.705 83.62) (end 184.925 86.84) (width 0.2) (layer "F.Cu") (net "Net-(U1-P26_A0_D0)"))
 (segment (start 155.35 85.46) (end 156.79 84.02) (width 0.2) (layer "F.Cu") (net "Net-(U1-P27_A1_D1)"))
 (segment (start 184.09 89.38) (end 184.925 89.38) (width 0.2) (layer "F.Cu") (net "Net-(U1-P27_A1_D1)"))
 (segment (start 178.73 84.02) (end 184.09 89.38) (width 0.2) (layer "F.Cu") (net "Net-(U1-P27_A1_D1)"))
 (segment (start 156.79 84.02) (end 178.73 84.02) (width 0.2) (layer "F.Cu") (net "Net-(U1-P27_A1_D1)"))
 (segment (start 175.04 85.42) (end 181.54 91.92) (width 0.2) (layer "F.Cu") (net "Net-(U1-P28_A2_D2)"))
 (segment (start 181.54 91.92) (end 184.925 91.92) (width 0.2) (layer "F.Cu") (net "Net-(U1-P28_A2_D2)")))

